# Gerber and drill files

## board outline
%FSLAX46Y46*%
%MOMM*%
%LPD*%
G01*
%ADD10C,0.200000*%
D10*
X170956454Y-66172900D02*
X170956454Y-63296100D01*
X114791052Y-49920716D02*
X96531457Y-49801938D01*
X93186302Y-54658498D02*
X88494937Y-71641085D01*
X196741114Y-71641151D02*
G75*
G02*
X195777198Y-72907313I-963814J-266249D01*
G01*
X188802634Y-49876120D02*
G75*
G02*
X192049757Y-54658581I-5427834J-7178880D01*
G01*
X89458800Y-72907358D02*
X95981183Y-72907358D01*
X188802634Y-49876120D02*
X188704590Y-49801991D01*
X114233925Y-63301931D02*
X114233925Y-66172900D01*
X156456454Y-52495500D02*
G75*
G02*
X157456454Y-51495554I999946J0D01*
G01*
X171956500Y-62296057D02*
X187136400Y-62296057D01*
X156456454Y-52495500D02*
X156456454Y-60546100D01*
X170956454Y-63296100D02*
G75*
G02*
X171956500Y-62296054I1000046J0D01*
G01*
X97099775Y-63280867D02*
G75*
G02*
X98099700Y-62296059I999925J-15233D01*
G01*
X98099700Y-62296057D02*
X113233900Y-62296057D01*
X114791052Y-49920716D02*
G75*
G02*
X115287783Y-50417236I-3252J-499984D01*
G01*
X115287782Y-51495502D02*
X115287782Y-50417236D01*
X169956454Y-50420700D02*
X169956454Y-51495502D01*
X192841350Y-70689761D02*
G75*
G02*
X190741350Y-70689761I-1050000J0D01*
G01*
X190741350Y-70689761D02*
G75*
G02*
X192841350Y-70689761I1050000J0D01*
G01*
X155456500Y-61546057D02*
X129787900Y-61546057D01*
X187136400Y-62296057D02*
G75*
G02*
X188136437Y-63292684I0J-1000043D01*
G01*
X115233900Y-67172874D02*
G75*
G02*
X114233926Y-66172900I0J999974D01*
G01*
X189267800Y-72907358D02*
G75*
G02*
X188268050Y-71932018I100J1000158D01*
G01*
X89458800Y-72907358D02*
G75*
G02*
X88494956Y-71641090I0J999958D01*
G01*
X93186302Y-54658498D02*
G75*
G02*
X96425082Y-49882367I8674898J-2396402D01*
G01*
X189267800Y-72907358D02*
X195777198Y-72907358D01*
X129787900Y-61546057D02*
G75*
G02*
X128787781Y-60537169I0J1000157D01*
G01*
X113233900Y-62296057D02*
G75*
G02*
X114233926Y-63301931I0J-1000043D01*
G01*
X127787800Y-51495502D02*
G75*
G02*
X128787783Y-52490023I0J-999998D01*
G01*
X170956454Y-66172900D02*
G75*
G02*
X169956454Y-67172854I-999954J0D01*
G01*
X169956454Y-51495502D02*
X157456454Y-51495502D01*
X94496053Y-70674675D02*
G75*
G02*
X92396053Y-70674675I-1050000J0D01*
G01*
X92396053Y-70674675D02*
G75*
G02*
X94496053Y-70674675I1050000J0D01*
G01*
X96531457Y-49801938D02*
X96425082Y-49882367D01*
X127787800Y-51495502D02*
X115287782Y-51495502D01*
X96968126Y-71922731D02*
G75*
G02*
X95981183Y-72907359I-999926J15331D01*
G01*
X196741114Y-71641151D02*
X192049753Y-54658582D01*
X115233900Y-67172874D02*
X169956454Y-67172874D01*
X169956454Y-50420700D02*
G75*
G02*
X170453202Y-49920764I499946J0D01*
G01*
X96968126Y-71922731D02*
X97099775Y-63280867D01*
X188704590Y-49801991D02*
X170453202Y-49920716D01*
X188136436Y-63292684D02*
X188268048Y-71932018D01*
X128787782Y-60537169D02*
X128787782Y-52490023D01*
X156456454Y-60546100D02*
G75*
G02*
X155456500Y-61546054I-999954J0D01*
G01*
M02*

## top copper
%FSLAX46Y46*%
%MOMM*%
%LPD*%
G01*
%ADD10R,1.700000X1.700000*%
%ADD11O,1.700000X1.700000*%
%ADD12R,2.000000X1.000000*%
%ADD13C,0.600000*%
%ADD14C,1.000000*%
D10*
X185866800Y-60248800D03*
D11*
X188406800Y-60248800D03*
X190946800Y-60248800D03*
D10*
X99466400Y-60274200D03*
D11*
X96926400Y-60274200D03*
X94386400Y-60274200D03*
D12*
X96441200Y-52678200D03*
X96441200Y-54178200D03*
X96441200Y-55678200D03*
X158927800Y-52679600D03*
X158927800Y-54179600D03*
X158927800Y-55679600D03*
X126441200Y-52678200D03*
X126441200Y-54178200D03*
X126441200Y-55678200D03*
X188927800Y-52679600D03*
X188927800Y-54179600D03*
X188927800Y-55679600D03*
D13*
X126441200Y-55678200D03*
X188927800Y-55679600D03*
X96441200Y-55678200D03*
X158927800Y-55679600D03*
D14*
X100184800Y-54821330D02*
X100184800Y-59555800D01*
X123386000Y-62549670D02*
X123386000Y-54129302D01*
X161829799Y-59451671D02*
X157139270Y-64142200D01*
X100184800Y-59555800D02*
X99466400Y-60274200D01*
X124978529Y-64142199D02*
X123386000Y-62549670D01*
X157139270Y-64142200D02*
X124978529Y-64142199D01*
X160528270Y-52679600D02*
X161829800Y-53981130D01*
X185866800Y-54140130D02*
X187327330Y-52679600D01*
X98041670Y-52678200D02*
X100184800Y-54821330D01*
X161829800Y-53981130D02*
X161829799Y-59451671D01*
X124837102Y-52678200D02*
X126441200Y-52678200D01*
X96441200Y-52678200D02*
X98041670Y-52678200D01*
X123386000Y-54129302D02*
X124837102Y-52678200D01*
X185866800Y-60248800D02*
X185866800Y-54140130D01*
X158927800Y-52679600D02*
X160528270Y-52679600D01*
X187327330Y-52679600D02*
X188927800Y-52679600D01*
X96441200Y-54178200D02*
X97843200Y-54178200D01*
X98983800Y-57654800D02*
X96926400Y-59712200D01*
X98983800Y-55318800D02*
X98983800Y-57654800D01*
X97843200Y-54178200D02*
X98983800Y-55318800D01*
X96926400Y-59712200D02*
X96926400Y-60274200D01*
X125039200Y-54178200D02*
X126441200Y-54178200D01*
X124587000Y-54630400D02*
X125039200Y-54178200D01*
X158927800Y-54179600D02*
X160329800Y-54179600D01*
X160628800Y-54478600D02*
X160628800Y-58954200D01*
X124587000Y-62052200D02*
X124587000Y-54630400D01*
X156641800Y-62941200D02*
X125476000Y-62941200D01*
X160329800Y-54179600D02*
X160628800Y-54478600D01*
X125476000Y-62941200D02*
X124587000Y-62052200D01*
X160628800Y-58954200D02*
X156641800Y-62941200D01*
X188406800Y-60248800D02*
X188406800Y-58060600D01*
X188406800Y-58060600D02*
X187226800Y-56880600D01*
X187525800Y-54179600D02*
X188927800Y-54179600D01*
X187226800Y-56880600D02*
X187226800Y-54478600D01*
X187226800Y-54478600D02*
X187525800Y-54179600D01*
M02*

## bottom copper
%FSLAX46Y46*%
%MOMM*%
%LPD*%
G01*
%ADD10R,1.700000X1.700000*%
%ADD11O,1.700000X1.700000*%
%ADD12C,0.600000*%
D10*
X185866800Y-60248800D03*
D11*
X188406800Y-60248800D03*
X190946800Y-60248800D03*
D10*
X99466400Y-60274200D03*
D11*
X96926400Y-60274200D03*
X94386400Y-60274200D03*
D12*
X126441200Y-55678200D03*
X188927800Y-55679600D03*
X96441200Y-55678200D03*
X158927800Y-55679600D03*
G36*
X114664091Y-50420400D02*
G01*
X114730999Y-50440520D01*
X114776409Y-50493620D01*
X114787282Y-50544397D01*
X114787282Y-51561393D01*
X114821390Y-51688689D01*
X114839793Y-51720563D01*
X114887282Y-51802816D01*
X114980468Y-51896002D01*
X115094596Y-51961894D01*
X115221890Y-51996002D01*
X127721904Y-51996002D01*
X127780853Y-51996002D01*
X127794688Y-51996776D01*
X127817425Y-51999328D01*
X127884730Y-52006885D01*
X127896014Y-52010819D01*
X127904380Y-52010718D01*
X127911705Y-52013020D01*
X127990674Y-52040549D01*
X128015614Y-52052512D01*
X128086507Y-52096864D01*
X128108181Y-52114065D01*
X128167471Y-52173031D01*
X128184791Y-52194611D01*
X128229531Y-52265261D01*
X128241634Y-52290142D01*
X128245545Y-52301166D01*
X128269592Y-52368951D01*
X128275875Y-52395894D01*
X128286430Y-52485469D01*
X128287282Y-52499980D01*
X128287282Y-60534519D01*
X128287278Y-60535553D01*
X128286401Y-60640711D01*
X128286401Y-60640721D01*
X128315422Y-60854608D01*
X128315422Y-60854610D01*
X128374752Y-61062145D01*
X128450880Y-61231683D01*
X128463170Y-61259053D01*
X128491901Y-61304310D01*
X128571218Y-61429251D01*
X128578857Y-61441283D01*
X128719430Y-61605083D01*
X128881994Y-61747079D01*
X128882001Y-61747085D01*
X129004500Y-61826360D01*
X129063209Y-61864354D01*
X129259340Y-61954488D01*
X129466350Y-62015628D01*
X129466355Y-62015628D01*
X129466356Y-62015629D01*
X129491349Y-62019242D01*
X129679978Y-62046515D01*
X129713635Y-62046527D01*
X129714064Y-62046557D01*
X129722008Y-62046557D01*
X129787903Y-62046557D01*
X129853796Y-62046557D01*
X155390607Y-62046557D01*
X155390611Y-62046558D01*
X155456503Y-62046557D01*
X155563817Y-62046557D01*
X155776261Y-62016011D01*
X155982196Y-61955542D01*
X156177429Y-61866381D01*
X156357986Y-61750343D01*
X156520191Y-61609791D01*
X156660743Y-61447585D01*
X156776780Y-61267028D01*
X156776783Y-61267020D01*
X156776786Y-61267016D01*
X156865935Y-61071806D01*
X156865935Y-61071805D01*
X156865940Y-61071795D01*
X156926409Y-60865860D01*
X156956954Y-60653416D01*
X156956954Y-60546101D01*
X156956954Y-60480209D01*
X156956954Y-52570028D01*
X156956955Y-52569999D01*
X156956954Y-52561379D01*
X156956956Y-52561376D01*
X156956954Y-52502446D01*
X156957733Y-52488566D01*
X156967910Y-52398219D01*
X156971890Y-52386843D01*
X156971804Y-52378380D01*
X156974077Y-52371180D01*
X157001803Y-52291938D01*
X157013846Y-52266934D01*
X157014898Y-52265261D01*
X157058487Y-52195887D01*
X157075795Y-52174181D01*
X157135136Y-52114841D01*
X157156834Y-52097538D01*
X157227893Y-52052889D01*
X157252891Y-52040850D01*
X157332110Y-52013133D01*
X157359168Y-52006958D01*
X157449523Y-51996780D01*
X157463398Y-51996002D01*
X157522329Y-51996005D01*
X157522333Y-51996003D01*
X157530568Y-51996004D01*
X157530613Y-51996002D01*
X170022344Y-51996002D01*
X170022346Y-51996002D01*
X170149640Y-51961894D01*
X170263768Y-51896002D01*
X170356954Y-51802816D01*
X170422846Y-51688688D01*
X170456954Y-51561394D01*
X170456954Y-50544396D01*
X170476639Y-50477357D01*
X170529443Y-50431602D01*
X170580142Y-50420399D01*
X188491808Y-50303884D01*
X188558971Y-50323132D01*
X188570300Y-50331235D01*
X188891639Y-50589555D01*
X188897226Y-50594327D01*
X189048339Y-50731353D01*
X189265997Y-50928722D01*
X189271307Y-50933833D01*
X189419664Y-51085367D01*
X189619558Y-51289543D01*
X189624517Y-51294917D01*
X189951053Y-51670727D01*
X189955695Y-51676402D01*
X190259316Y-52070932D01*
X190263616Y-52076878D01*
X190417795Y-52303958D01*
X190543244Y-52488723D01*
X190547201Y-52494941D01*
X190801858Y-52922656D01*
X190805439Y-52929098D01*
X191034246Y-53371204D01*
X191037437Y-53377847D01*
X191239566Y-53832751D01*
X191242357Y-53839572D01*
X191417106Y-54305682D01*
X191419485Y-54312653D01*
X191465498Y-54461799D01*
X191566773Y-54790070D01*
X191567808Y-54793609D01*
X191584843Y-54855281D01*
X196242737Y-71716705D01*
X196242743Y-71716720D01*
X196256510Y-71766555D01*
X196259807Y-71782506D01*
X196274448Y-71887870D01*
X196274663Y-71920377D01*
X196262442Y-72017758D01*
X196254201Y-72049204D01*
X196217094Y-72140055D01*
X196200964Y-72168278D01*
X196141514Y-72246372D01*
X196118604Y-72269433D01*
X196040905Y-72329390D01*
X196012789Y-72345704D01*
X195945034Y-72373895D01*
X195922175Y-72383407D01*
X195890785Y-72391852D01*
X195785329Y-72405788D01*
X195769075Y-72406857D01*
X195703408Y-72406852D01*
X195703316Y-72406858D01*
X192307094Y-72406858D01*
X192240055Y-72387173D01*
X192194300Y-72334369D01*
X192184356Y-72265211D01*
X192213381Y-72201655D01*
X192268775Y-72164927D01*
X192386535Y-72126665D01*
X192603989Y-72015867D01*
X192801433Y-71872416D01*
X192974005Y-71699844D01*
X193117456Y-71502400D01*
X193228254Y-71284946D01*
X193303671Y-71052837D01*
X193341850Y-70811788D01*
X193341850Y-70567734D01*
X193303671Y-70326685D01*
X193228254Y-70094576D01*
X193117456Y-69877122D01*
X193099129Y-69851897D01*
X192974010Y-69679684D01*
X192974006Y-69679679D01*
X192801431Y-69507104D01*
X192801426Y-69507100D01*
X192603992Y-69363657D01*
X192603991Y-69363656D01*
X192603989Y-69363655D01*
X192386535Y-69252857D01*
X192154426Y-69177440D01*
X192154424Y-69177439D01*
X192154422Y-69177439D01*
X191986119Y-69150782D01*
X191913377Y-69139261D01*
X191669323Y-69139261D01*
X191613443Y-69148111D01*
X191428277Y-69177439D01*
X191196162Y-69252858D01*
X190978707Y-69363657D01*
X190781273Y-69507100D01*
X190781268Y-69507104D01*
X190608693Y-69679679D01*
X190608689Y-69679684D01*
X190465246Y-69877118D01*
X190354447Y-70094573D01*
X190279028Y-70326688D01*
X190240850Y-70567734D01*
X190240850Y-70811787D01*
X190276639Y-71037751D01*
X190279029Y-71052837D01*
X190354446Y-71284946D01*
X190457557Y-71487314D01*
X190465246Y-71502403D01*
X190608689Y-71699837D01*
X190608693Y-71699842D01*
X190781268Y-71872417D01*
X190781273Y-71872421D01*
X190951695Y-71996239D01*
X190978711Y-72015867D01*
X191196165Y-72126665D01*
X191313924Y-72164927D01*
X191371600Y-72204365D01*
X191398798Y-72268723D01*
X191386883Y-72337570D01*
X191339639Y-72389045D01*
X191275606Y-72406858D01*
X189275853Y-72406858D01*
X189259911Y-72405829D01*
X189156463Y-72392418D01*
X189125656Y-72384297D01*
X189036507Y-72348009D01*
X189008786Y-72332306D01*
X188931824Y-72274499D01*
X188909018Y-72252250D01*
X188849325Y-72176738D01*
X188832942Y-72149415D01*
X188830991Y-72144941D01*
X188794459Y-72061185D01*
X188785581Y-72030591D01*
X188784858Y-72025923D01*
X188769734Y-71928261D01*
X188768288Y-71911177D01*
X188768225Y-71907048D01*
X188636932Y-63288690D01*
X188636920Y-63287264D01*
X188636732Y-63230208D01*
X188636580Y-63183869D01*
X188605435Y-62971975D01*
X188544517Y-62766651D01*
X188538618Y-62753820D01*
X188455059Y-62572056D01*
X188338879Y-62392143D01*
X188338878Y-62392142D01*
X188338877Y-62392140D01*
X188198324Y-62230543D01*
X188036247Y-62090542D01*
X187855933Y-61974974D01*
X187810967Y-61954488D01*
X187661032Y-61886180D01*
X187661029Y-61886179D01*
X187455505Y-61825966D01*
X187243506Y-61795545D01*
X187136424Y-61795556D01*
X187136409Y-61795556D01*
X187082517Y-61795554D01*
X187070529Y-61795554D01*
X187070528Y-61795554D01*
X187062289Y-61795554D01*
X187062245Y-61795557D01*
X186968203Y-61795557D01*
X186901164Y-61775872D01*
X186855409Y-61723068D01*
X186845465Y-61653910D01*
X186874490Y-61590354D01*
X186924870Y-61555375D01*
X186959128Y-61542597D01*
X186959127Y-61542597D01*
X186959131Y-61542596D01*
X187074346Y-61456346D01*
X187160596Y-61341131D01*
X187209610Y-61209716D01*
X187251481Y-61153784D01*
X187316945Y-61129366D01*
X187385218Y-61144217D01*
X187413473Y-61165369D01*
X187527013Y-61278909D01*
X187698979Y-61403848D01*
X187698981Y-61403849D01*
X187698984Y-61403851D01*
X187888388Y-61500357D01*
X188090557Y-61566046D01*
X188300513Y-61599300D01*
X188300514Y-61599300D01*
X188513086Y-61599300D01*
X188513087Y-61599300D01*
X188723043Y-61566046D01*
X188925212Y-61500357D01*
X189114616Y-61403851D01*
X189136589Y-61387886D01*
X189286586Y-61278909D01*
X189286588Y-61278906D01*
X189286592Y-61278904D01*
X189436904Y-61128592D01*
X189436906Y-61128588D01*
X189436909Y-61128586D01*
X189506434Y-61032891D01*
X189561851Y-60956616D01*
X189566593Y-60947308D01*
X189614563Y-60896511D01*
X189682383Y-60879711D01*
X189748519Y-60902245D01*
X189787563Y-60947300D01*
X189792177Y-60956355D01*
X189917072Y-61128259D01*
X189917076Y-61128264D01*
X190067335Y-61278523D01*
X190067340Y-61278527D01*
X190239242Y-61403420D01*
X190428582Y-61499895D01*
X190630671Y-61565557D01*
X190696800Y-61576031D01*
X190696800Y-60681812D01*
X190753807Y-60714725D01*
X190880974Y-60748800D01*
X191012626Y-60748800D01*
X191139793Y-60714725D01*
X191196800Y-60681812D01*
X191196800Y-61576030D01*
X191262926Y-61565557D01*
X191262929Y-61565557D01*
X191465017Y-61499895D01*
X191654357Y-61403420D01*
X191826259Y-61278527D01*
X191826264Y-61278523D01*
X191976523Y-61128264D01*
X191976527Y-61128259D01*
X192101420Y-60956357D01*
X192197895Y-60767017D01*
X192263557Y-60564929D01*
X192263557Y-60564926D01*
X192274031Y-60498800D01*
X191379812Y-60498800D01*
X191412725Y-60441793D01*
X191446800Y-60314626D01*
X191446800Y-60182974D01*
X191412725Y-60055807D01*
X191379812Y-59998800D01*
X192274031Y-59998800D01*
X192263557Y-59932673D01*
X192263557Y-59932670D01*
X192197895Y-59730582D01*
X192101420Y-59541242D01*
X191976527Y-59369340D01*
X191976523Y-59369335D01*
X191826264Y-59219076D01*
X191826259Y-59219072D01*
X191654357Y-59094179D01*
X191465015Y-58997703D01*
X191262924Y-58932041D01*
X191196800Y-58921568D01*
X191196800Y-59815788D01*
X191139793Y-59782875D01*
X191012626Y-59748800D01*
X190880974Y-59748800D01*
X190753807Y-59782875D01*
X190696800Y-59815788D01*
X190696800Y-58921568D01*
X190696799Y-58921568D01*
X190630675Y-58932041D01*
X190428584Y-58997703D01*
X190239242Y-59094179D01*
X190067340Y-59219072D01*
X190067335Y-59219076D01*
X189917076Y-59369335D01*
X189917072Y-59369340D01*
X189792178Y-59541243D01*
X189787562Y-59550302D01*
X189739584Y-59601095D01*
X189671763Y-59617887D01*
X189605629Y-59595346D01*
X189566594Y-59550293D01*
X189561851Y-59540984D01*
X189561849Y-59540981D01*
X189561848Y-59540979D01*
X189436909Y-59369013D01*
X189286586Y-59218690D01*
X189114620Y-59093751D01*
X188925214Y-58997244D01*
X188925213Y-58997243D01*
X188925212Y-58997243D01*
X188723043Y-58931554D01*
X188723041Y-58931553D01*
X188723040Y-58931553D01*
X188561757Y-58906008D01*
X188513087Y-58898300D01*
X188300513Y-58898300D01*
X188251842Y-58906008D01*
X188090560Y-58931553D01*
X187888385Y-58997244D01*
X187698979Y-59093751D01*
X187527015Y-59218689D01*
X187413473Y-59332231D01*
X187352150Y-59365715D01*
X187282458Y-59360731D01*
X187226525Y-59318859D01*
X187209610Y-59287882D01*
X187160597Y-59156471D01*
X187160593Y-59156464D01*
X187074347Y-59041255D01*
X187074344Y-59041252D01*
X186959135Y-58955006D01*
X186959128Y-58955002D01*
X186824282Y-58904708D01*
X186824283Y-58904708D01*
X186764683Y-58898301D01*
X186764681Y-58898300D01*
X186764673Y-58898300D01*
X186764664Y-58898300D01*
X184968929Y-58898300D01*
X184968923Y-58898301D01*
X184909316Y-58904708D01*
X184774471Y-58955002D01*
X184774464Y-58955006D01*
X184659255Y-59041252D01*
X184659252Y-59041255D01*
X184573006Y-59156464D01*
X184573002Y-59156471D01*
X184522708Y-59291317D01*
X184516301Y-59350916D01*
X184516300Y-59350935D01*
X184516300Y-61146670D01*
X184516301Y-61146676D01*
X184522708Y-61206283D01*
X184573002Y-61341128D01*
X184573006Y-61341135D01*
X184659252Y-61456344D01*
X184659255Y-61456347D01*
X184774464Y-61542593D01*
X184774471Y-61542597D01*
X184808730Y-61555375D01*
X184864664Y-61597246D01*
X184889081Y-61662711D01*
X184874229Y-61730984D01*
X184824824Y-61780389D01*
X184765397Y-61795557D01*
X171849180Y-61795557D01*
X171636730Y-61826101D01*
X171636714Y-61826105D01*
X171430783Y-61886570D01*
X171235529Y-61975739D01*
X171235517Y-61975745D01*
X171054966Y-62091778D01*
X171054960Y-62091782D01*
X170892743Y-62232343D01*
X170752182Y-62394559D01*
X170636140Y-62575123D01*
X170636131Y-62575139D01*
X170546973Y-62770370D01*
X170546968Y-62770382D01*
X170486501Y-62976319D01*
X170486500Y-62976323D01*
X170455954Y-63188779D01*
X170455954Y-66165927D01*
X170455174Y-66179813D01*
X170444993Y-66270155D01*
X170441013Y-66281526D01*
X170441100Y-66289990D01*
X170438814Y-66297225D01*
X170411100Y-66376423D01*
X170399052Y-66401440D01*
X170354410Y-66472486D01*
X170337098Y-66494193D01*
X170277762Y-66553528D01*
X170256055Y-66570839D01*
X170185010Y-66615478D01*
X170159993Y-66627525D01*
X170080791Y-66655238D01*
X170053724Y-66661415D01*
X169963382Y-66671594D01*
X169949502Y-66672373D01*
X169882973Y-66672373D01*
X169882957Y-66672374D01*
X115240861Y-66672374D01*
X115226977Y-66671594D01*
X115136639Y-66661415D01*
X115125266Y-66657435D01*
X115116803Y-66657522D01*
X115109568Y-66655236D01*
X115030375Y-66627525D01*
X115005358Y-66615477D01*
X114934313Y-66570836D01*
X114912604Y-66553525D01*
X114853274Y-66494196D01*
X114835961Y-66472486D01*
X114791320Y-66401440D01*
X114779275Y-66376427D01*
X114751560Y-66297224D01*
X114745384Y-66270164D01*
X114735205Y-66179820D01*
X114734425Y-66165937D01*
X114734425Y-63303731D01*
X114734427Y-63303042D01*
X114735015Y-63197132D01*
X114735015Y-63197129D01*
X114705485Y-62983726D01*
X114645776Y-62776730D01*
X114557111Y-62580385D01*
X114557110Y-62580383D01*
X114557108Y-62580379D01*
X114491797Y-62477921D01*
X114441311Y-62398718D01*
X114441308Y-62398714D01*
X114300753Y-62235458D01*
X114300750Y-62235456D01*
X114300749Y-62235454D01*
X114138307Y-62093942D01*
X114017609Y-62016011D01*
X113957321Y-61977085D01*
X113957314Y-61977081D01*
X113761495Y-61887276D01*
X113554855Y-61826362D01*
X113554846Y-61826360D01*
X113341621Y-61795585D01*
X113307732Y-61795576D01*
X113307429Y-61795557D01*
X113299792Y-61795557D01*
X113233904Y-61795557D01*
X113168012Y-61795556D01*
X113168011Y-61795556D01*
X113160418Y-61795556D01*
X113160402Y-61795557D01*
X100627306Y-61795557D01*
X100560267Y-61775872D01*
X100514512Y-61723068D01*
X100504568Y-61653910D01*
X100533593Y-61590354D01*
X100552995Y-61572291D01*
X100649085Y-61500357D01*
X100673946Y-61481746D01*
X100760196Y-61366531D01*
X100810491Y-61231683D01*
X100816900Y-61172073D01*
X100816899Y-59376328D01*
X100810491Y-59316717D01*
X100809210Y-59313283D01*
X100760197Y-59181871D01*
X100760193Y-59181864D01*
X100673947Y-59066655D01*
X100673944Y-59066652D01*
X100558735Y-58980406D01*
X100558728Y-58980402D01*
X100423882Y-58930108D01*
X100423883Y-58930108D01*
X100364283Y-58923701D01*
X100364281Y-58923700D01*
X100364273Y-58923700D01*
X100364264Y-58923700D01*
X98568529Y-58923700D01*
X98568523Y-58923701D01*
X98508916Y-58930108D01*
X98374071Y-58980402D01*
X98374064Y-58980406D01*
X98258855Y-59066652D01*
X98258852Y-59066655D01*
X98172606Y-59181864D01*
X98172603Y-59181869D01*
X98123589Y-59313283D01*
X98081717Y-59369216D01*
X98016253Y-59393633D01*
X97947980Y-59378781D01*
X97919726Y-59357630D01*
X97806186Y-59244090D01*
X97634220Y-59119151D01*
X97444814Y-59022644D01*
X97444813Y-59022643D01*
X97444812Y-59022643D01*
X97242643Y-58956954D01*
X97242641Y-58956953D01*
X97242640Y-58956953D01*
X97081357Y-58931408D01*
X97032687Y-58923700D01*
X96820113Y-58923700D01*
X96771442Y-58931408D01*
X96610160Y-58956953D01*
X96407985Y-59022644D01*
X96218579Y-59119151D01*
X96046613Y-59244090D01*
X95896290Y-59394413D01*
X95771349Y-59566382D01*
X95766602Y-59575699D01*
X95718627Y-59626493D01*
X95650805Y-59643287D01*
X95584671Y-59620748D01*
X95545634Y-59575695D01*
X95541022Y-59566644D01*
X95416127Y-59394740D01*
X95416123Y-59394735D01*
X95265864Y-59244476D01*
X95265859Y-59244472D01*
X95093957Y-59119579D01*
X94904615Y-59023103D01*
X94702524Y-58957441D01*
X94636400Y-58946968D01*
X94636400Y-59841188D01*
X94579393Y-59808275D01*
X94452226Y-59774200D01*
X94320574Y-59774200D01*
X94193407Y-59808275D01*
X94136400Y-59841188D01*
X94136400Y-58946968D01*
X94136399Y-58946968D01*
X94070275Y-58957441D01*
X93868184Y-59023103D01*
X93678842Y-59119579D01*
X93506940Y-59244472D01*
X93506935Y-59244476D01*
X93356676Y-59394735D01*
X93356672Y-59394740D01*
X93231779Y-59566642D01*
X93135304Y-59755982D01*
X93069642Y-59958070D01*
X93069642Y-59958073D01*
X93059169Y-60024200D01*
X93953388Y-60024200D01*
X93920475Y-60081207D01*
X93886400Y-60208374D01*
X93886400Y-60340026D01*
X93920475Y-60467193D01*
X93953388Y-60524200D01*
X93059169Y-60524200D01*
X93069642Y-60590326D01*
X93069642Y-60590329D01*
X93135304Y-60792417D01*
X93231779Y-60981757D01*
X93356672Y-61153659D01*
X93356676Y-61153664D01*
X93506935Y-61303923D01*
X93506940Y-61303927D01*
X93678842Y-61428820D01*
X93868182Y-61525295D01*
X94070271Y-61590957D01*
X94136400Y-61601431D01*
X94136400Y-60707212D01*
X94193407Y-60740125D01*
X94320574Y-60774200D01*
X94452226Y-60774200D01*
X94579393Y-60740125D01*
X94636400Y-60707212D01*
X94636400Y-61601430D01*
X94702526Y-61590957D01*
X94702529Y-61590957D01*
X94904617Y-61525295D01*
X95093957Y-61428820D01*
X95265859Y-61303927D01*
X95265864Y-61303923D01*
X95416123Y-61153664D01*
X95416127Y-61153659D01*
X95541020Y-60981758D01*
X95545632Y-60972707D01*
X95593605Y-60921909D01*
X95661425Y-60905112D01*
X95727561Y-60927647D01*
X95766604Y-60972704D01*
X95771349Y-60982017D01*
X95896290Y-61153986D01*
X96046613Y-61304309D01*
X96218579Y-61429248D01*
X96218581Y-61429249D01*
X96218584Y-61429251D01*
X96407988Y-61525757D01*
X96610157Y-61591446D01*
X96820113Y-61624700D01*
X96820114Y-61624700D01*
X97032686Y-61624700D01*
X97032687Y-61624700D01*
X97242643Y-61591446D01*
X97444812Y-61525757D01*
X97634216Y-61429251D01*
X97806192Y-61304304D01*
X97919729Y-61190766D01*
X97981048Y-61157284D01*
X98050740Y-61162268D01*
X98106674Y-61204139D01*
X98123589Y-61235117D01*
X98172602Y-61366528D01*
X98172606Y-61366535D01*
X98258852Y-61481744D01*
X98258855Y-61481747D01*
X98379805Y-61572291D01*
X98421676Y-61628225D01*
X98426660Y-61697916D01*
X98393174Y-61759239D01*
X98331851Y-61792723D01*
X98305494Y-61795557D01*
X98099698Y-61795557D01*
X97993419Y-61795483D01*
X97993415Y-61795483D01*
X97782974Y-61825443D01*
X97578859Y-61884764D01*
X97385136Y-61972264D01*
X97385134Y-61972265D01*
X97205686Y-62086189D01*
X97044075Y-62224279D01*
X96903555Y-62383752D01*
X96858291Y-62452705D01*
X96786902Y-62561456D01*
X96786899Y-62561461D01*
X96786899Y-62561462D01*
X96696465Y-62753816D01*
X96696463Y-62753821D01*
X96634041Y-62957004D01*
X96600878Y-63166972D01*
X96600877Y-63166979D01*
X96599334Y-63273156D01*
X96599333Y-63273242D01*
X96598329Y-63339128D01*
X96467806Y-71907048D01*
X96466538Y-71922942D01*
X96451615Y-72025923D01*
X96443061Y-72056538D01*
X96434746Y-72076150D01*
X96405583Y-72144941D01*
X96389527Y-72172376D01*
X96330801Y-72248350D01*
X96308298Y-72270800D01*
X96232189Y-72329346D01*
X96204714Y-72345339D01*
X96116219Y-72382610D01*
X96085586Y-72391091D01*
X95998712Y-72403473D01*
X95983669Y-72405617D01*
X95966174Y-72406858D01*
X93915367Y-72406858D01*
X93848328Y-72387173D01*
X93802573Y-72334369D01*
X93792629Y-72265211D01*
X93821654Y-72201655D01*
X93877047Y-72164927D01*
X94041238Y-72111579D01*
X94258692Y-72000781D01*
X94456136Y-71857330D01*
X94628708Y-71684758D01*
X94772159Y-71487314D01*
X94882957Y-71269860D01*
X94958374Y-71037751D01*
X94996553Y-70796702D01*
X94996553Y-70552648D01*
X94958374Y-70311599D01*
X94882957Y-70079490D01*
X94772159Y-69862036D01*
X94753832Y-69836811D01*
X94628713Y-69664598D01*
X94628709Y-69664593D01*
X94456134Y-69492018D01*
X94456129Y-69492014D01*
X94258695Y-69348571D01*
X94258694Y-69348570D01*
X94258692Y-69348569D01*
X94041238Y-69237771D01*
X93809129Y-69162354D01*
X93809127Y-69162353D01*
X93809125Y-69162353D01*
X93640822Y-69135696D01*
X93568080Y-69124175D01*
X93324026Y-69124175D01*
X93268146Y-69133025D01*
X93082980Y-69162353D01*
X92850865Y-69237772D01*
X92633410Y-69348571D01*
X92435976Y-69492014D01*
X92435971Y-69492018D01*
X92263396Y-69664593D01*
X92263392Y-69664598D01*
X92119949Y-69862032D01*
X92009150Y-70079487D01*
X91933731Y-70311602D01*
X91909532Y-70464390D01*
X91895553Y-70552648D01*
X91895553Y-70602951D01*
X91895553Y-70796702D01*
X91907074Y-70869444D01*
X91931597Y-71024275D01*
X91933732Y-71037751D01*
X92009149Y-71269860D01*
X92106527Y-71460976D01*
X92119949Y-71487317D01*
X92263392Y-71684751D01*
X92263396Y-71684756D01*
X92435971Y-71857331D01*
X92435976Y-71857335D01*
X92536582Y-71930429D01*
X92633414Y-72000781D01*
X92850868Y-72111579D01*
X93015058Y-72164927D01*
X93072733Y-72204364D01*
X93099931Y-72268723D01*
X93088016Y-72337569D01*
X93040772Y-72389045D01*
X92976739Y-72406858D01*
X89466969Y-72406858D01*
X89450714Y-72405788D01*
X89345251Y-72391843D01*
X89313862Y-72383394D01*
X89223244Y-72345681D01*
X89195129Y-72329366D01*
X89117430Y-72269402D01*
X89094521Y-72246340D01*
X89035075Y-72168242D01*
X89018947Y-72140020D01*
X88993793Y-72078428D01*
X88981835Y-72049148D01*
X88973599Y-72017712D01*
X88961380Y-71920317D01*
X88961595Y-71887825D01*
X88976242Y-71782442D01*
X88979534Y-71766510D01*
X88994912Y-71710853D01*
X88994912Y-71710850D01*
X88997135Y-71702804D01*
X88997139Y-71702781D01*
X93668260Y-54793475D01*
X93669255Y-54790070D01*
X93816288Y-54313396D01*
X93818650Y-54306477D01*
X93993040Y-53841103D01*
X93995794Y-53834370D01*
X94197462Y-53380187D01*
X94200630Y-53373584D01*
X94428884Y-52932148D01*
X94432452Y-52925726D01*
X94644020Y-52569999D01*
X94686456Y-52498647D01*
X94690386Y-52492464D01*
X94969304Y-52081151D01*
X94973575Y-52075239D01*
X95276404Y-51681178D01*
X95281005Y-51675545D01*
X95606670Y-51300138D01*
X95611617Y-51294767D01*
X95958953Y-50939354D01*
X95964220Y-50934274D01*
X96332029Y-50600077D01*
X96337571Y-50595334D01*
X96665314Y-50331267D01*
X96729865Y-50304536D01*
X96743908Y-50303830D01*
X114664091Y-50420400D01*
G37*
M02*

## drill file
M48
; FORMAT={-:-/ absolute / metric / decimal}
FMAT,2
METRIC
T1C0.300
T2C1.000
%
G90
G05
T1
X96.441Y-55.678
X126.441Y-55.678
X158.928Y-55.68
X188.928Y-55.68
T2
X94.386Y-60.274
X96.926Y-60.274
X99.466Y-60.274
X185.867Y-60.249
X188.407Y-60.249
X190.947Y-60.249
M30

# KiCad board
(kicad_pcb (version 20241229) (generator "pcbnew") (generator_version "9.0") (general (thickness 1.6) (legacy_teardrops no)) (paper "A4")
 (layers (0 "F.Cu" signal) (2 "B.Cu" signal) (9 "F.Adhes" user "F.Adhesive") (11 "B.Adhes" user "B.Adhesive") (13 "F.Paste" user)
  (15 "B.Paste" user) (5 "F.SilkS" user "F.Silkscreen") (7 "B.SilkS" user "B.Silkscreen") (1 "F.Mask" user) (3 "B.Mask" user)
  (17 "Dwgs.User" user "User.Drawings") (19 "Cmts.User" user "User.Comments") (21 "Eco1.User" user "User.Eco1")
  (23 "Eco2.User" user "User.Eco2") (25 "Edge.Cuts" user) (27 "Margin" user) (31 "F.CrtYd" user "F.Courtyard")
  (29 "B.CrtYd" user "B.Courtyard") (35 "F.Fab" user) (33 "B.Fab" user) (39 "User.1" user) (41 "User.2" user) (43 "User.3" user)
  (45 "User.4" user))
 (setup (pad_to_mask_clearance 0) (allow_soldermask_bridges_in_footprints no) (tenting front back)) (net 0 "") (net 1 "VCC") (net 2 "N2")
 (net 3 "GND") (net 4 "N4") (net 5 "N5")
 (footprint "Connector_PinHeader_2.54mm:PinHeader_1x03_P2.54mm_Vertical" (layer "F.Cu") (at 185.8668 60.2488 90)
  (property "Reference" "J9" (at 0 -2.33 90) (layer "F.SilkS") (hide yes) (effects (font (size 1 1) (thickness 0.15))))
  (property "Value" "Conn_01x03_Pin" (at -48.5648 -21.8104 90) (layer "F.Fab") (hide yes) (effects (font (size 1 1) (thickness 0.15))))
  (pad "1" thru_hole rect (at 0 0 90) (size 1.7 1.7) (drill 1) (layers "*.Cu" "*.Mask") (remove_unused_layers no) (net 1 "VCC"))
  (pad "2" thru_hole oval (at 0 2.54 90) (size 1.7 1.7) (drill 1) (layers "*.Cu" "*.Mask") (remove_unused_layers no) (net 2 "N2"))
  (pad "3" thru_hole oval (at 0 5.08 90) (size 1.7 1.7) (drill 1) (layers "*.Cu" "*.Mask") (remove_unused_layers no) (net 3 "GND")))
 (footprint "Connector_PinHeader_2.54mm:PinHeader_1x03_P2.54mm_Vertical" (layer "F.Cu") (at 99.4664 60.2742 -90)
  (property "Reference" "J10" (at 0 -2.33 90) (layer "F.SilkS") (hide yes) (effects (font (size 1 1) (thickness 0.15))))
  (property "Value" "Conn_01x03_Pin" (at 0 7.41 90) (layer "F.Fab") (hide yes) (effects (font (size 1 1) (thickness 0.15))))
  (pad "1" thru_hole rect (at 0 0 270) (size 1.7 1.7) (drill 1) (layers "*.Cu" "*.Mask") (remove_unused_layers no) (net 1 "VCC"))
  (pad "2" thru_hole oval (at 0 2.54 270) (size 1.7 1.7) (drill 1) (layers "*.Cu" "*.Mask") (remove_unused_layers no) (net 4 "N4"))
  (pad "3" thru_hole oval (at 0 5.08 270) (size 1.7 1.7) (drill 1) (layers "*.Cu" "*.Mask") (remove_unused_layers no) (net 3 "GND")))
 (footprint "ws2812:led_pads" (layer "F.Cu") (at 96.4412 54.1782 -90)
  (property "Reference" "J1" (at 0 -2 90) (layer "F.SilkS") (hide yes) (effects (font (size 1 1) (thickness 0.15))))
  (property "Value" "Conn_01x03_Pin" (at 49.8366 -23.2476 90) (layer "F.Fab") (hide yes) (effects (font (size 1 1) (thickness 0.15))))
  (pad "1" smd rect (at -1.5 0 270) (size 1 2) (layers "F.Cu" "F.Mask" "F.Paste") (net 1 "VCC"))
  (pad "2" smd rect (at 0 0 270) (size 1 2) (layers "F.Cu" "F.Mask" "F.Paste") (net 4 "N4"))
  (pad "3" smd rect (at 1.5 0 270) (size 1 2) (layers "F.Cu" "F.Mask" "F.Paste") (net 3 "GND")))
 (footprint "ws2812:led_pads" (layer "F.Cu") (at 158.9278 54.1796 -90)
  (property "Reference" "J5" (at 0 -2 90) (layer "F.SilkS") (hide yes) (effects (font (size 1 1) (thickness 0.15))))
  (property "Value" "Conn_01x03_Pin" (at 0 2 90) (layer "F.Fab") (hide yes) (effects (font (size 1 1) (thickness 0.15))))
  (pad "1" smd rect (at -1.5 0 270) (size 1 2) (layers "F.Cu" "F.Mask" "F.Paste") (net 1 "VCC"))
  (pad "2" smd rect (at 0 0 270) (size 1 2) (layers "F.Cu" "F.Mask" "F.Paste") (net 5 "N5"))
  (pad "3" smd rect (at 1.5 0 270) (size 1 2) (layers "F.Cu" "F.Mask" "F.Paste") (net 3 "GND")))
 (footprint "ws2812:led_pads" (layer "F.Cu") (at 126.4412 54.1782 -90)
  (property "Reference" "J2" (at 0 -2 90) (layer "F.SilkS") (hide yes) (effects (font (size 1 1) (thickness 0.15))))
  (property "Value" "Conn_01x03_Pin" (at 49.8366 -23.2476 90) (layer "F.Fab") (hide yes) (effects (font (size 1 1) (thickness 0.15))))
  (pad "1" smd rect (at -1.5 0 270) (size 1 2) (layers "F.Cu" "F.Mask" "F.Paste") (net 1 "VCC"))
  (pad "2" smd rect (at 0 0 270) (size 1 2) (layers "F.Cu" "F.Mask" "F.Paste") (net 5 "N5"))
  (pad "3" smd rect (at 1.5 0 270) (size 1 2) (layers "F.Cu" "F.Mask" "F.Paste") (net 3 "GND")))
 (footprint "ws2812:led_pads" (layer "F.Cu") (at 188.9278 54.1796 -90)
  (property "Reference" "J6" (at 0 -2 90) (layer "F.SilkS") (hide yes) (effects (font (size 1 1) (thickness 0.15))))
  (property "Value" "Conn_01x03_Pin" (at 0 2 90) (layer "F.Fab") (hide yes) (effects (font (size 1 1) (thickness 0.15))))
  (pad "1" smd rect (at -1.5 0 270) (size 1 2) (layers "F.Cu" "F.Mask" "F.Paste") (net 1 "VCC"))
  (pad "2" smd rect (at 0 0 270) (size 1 2) (layers "F.Cu" "F.Mask" "F.Paste") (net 2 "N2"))
  (pad "3" smd rect (at 1.5 0 270) (size 1 2) (layers "F.Cu" "F.Mask" "F.Paste") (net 3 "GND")))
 (gr_line (start 170.956454 66.1729) (end 170.956454 63.2961) (stroke (width 0.2) (type default)) (layer "Edge.Cuts"))
 (gr_line (start 114.791052 49.920716) (end 96.531457 49.801938) (stroke (width 0.2) (type default)) (layer "Edge.Cuts"))
 (gr_line (start 93.186302 54.658498) (end 88.494937 71.641085) (stroke (width 0.2) (type default)) (layer "Edge.Cuts"))
 (gr_arc (start 196.741114 71.641151) (mid 196.572918 72.513083) (end 195.777198 72.907358) (stroke (width 0.2) (type default))
  (layer "Edge.Cuts"))
 (gr_arc (start 188.802634 49.87612) (mid 190.820615 51.999553) (end 192.049753 54.658582) (stroke (width 0.2) (type default))
  (layer "Edge.Cuts"))
 (gr_line (start 89.4588 72.907358) (end 95.981183 72.907358) (stroke (width 0.2) (type default)) (layer "Edge.Cuts"))
 (gr_line (start 188.802634 49.87612) (end 188.70459 49.801991) (stroke (width 0.2) (type default)) (layer "Edge.Cuts"))
 (gr_line (start 114.233925 63.301931) (end 114.233925 66.1729) (stroke (width 0.2) (type default)) (layer "Edge.Cuts"))
 (gr_arc (start 156.456454 52.4955) (mid 156.749344 51.788378) (end 157.456454 51.495502) (stroke (width 0.2) (type default))
  (layer "Edge.Cuts"))
 (gr_line (start 171.9565 62.296057) (end 187.1364 62.296057) (stroke (width 0.2) (type default)) (layer "Edge.Cuts"))
 (gr_line (start 156.456454 52.4955) (end 156.456454 60.5461) (stroke (width 0.2) (type default)) (layer "Edge.Cuts"))
 (gr_arc (start 170.956454 63.2961) (mid 171.24936 62.588962) (end 171.9565 62.296057) (stroke (width 0.2) (type default))
  (layer "Edge.Cuts"))
 (gr_arc (start 97.099775 63.280867) (mid 97.397972 62.583598) (end 98.0997 62.296057) (stroke (width 0.2) (type default))
  (layer "Edge.Cuts"))
 (gr_line (start 98.0997 62.296057) (end 113.2339 62.296057) (stroke (width 0.2) (type default)) (layer "Edge.Cuts"))
 (gr_arc (start 114.791052 49.920716) (mid 115.142493 50.068298) (end 115.287782 50.417236) (stroke (width 0.2) (type default))
  (layer "Edge.Cuts"))
 (gr_line (start 115.287782 51.495502) (end 115.287782 50.417236) (stroke (width 0.2) (type default)) (layer "Edge.Cuts"))
 (gr_line (start 169.956454 50.4207) (end 169.956454 51.495502) (stroke (width 0.2) (type default)) (layer "Edge.Cuts"))
 (gr_circle (center 191.79135 70.689761) (end 192.84135 70.689761) (stroke (width 0.2) (type default)) (fill no) (layer "Edge.Cuts"))
 (gr_line (start 155.4565 61.546057) (end 129.7879 61.546057) (stroke (width 0.2) (type default)) (layer "Edge.Cuts"))
 (gr_arc (start 187.1364 62.296057) (mid 187.838106 62.583573) (end 188.136436 63.292684) (stroke (width 0.2) (type default))
  (layer "Edge.Cuts"))
 (gr_arc (start 115.2339 67.172874) (mid 114.526811 66.879988) (end 114.233925 66.1729) (stroke (width 0.2) (type default))
  (layer "Edge.Cuts"))
 (gr_arc (start 189.2678 72.907358) (mid 188.566109 72.619823) (end 188.268048 71.932018) (stroke (width 0.2) (type default))
  (layer "Edge.Cuts"))
 (gr_arc (start 89.4588 72.907358) (mid 88.66313 72.513061) (end 88.494937 71.641085) (stroke (width 0.2) (type default))
  (layer "Edge.Cuts"))
 (gr_arc (start 93.186302 54.658498) (mid 94.415433 51.999496) (end 96.425082 49.882367) (stroke (width 0.2) (type default))
  (layer "Edge.Cuts"))
 (gr_line (start 189.2678 72.907358) (end 195.777198 72.907358) (stroke (width 0.2) (type default)) (layer "Edge.Cuts"))
 (gr_arc (start 129.7879 61.546057) (mid 129.080702 61.253155) (end 128.787782 60.537169) (stroke (width 0.2) (type default))
  (layer "Edge.Cuts"))
 (gr_arc (start 113.2339 62.296057) (mid 113.941031 62.588956) (end 114.233925 63.301931) (stroke (width 0.2) (type default))
  (layer "Edge.Cuts"))
 (gr_arc (start 127.7878 51.495502) (mid 128.4949 51.788389) (end 128.787782 52.490023) (stroke (width 0.2) (type default))
  (layer "Edge.Cuts"))
 (gr_arc (start 170.956454 66.1729) (mid 170.663567 66.879981) (end 169.956454 67.172874) (stroke (width 0.2) (type default))
  (layer "Edge.Cuts"))
 (gr_line (start 169.956454 51.495502) (end 157.456454 51.495502) (stroke (width 0.2) (type default)) (layer "Edge.Cuts"))
 (gr_circle (center 93.446053 70.674675) (end 94.496053 70.674675) (stroke (width 0.2) (type default)) (fill no) (layer "Edge.Cuts"))
 (gr_line (start 96.531457 49.801938) (end 96.425082 49.882367) (stroke (width 0.2) (type default)) (layer "Edge.Cuts"))
 (gr_line (start 127.7878 51.495502) (end 115.287782 51.495502) (stroke (width 0.2) (type default)) (layer "Edge.Cuts"))
 (gr_arc (start 96.968126 71.922731) (mid 96.669962 72.619872) (end 95.981183 72.907358) (stroke (width 0.2) (type default))
  (layer "Edge.Cuts"))
 (gr_line (start 196.741114 71.641151) (end 192.049753 54.658582) (stroke (width 0.2) (type default)) (layer "Edge.Cuts"))
 (gr_line (start 115.2339 67.172874) (end 169.956454 67.172874) (stroke (width 0.2) (type default)) (layer "Edge.Cuts"))
 (gr_arc (start 169.956454 50.4207) (mid 170.101748 50.068284) (end 170.453202 49.920716) (stroke (width 0.2) (type default))
  (layer "Edge.Cuts"))
 (gr_line (start 96.968126 71.922731) (end 97.099775 63.280867) (stroke (width 0.2) (type default)) (layer "Edge.Cuts"))
 (gr_line (start 188.70459 49.801991) (end 170.453202 49.920716) (stroke (width 0.2) (type default)) (layer "Edge.Cuts"))
 (gr_line (start 188.136436 63.292684) (end 188.268048 71.932018) (stroke (width 0.2) (type default)) (layer "Edge.Cuts"))
 (gr_line (start 128.787782 60.537169) (end 128.787782 52.490023) (stroke (width 0.2) (type default)) (layer "Edge.Cuts"))
 (gr_arc (start 156.456454 60.5461) (mid 156.163573 61.253175) (end 155.4565 61.546057) (stroke (width 0.2) (type default))
  (layer "Edge.Cuts"))
 (via (at 126.4412 55.6782) (size 0.6) (drill 0.3) (layers "F.Cu" "B.Cu") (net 3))
 (via (at 188.9278 55.6796) (size 0.6) (drill 0.3) (layers "F.Cu" "B.Cu") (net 3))
 (via (at 96.4412 55.6782) (size 0.6) (drill 0.3) (layers "F.Cu" "B.Cu") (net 3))
 (via (at 158.9278 55.6796) (size 0.6) (drill 0.3) (layers "F.Cu" "B.Cu") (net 3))
 (segment (start 100.1848 54.82133) (end 100.1848 59.5558) (width 1) (layer "F.Cu") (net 1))
 (segment (start 123.386 62.54967) (end 123.386 54.129302) (width 1) (layer "F.Cu") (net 1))
 (segment (start 161.829799 59.451671) (end 157.13927 64.1422) (width 1) (layer "F.Cu") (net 1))
 (segment (start 100.1848 59.5558) (end 99.4664 60.2742) (width 1) (layer "F.Cu") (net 1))
 (segment (start 124.978529 64.142199) (end 123.386 62.54967) (width 1) (layer "F.Cu") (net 1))
 (segment (start 157.13927 64.1422) (end 124.978529 64.142199) (width 1) (layer "F.Cu") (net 1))
 (segment (start 160.52827 52.6796) (end 161.8298 53.98113) (width 1) (layer "F.Cu") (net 1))
 (segment (start 185.8668 54.14013) (end 187.32733 52.6796) (width 1) (layer "F.Cu") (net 1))
 (segment (start 98.04167 52.6782) (end 100.1848 54.82133) (width 1) (layer "F.Cu") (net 1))
 (segment (start 161.8298 53.98113) (end 161.829799 59.451671) (width 1) (layer "F.Cu") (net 1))
 (segment (start 124.837102 52.6782) (end 126.4412 52.6782) (width 1) (layer "F.Cu") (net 1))
 (segment (start 96.4412 52.6782) (end 98.04167 52.6782) (width 1) (layer "F.Cu") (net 1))
 (segment (start 123.386 54.129302) (end 124.837102 52.6782) (width 1) (layer "F.Cu") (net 1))
 (segment (start 185.8668 60.2488) (end 185.8668 54.14013) (width 1) (layer "F.Cu") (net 1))
 (segment (start 158.9278 52.6796) (end 160.52827 52.6796) (width 1) (layer "F.Cu") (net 1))
 (segment (start 187.32733 52.6796) (end 188.9278 52.6796) (width 1) (layer "F.Cu") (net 1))
 (segment (start 96.4412 54.1782) (end 97.8432 54.1782) (width 1) (layer "F.Cu") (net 4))
 (segment (start 98.9838 57.6548) (end 96.9264 59.7122) (width 1) (layer "F.Cu") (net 4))
 (segment (start 98.9838 55.3188) (end 98.9838 57.6548) (width 1) (layer "F.Cu") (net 4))
 (segment (start 97.8432 54.1782) (end 98.9838 55.3188) (width 1) (layer "F.Cu") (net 4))
 (segment (start 96.9264 59.7122) (end 96.9264 60.2742) (width 1) (layer "F.Cu") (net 4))
 (segment (start 125.0392 54.1782) (end 126.4412 54.1782) (width 1) (layer "F.Cu") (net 5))
 (segment (start 124.587 54.6304) (end 125.0392 54.1782) (width 1) (layer "F.Cu") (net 5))
 (segment (start 158.9278 54.1796) (end 160.3298 54.1796) (width 1) (layer "F.Cu") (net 5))
 (segment (start 160.6288 54.4786) (end 160.6288 58.9542) (width 1) (layer "F.Cu") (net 5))
 (segment (start 124.587 62.0522) (end 124.587 54.6304) (width 1) (layer "F.Cu") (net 5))
 (segment (start 156.6418 62.9412) (end 125.476 62.9412) (width 1) (layer "F.Cu") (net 5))
 (segment (start 160.3298 54.1796) (end 160.6288 54.4786) (width 1) (layer "F.Cu") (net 5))
 (segment (start 125.476 62.9412) (end 124.587 62.0522) (width 1) (layer "F.Cu") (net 5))
 (segment (start 160.6288 58.9542) (end 156.6418 62.9412) (width 1) (layer "F.Cu") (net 5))
 (segment (start 188.4068 60.2488) (end 188.4068 58.0606) (width 1) (layer "F.Cu") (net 2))
 (segment (start 188.4068 58.0606) (end 187.2268 56.8806) (width 1) (layer "F.Cu") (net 2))
 (segment (start 187.5258 54.1796) (end 188.9278 54.1796) (width 1) (layer "F.Cu") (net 2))
 (segment (start 187.2268 56.8806) (end 187.2268 54.4786) (width 1) (layer "F.Cu") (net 2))
 (segment (start 187.2268 54.4786) (end 187.5258 54.1796) (width 1) (layer "F.Cu") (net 2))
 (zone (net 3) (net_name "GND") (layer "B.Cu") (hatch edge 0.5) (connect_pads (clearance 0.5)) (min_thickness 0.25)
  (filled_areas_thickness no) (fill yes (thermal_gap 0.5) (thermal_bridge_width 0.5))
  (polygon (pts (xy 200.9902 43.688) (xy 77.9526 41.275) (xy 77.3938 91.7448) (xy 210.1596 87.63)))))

